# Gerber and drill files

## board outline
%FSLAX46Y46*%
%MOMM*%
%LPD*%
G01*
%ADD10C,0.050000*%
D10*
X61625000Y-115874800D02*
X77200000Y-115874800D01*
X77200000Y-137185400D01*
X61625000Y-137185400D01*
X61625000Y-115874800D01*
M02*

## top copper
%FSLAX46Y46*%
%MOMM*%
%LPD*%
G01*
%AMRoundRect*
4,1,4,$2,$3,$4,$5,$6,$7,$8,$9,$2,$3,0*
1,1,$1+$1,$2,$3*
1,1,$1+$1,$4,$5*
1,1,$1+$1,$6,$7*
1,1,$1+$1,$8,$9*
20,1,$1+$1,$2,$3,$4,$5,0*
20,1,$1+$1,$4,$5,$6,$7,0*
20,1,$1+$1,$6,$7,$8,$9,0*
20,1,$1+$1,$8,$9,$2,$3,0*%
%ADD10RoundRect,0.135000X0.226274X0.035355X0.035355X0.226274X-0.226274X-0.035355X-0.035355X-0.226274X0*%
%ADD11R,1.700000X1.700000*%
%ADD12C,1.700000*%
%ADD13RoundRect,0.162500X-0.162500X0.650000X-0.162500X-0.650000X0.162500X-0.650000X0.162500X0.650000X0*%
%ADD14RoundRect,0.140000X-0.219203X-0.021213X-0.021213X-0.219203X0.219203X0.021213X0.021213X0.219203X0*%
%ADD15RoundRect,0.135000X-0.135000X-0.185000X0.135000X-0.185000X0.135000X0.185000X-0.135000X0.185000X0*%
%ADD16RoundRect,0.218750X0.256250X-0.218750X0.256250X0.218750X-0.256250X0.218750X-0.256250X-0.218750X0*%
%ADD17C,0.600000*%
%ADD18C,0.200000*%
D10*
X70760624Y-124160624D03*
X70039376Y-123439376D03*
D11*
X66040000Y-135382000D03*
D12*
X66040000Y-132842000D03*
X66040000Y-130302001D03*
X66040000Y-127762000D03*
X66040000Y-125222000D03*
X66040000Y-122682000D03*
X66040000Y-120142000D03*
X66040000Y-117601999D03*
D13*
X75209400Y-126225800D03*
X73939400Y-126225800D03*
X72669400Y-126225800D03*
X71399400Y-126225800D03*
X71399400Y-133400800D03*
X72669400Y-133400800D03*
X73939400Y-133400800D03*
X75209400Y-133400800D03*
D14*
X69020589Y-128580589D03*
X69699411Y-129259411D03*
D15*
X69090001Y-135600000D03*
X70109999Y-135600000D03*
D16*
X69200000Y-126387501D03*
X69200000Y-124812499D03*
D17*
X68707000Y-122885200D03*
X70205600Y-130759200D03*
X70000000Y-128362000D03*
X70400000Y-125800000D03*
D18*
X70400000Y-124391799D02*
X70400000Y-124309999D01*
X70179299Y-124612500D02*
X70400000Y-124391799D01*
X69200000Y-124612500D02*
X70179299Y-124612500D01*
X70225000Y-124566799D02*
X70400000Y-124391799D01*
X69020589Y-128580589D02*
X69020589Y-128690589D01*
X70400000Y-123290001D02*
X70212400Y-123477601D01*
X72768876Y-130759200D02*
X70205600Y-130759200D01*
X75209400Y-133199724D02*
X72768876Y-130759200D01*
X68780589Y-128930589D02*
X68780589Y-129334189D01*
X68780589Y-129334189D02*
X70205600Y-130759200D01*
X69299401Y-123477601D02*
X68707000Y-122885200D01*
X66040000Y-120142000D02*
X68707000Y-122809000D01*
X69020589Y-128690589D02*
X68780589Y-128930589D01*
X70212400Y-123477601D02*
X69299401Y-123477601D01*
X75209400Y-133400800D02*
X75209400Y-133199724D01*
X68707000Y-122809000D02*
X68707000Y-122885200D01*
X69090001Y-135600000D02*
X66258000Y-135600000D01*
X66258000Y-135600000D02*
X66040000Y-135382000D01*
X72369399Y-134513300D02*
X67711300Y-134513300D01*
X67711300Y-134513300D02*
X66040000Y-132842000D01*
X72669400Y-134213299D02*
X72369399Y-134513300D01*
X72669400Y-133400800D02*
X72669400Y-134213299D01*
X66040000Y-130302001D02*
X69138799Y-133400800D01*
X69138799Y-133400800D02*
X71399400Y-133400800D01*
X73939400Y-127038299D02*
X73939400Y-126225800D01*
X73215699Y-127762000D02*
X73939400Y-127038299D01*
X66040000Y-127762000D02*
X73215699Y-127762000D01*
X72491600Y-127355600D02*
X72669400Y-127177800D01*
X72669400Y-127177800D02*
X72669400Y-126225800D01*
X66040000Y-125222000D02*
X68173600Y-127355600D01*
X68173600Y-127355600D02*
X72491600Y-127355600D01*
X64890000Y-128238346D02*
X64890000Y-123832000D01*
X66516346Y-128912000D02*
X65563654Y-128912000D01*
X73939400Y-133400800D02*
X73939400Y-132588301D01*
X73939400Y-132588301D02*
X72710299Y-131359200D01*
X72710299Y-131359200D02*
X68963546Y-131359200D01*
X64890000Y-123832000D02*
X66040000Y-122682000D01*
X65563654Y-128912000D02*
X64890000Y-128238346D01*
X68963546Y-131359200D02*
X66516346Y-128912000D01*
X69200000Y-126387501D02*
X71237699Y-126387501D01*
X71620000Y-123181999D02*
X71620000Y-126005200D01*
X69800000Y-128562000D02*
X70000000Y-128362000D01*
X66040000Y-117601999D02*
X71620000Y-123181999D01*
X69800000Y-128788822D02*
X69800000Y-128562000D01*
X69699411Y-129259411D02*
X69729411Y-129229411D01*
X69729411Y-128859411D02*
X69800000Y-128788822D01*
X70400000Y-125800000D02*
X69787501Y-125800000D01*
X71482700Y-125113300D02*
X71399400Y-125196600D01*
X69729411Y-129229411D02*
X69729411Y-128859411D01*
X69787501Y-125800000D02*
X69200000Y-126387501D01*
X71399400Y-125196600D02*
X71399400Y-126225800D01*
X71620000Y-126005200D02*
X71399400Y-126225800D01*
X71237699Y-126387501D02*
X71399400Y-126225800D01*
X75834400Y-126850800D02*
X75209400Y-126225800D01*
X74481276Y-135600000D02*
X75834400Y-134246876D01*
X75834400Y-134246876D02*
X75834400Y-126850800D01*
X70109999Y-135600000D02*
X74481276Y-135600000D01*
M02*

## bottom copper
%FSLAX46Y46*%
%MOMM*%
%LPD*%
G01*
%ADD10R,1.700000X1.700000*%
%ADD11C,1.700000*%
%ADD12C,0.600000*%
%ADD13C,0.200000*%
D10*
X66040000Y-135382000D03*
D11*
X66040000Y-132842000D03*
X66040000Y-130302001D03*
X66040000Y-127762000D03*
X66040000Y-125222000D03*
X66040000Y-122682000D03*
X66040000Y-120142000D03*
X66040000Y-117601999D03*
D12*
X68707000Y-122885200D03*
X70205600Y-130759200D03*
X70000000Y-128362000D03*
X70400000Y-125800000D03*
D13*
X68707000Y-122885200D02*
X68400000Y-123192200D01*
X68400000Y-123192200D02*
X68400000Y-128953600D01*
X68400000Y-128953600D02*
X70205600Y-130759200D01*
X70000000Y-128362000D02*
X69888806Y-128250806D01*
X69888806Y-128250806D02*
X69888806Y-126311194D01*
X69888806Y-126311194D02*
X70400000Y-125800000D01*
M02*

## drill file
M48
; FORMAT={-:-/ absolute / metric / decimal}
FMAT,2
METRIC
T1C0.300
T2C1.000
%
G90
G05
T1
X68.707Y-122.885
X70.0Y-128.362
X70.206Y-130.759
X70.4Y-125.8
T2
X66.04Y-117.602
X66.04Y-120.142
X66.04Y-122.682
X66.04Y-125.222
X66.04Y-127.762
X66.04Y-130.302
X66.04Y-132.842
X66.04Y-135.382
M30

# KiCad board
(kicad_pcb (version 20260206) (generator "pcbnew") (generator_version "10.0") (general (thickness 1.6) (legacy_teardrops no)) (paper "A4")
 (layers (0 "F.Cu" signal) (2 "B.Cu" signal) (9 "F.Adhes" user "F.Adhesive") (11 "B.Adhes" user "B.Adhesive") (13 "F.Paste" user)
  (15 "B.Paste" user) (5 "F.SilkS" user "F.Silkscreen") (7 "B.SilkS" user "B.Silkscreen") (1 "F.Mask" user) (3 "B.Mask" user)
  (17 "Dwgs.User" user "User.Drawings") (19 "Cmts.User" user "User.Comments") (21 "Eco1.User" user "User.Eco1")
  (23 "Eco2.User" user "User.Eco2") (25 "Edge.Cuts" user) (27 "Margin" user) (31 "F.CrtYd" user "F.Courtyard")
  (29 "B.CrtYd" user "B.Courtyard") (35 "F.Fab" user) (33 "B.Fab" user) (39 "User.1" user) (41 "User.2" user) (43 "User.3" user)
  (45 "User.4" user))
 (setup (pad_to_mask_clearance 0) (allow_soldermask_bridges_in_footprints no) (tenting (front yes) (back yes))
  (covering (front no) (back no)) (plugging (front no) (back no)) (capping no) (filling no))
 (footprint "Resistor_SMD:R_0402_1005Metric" (layer "F.Cu") (at 70.4 123.8 135)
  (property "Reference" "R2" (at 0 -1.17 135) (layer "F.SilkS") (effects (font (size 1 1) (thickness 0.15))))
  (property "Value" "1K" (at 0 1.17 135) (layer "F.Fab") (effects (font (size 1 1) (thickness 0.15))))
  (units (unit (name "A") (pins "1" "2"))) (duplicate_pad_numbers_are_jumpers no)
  (pad "1" smd roundrect (at -0.509999 0 135) (size 0.54 0.64) (layers "F.Cu" "F.Mask" "F.Paste") (roundrect_rratio 0.25) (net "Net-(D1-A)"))
  (pad "2" smd roundrect (at 0.509999 0 135) (size 0.54 0.64) (layers "F.Cu" "F.Mask" "F.Paste") (roundrect_rratio 0.25) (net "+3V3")))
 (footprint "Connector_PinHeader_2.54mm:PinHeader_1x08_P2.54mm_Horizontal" (layer "F.Cu") (at 66.04 135.382 180)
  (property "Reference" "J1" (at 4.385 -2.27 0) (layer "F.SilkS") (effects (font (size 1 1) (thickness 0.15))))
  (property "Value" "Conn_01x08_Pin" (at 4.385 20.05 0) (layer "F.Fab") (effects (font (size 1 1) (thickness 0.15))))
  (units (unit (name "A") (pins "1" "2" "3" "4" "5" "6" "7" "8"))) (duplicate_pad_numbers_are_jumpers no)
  (pad "1" thru_hole rect (at 0 0 180) (size 1.7 1.7) (drill 1) (layers "*.Cu" "*.Mask") (remove_unused_layers no) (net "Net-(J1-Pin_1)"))
  (pad "2" thru_hole circle (at 0 2.54 180) (size 1.7 1.7) (drill 1) (layers "*.Cu" "*.Mask") (remove_unused_layers no)
   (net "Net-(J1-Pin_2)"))
  (pad "3" thru_hole circle (at 0 5.079999 180) (size 1.7 1.7) (drill 1) (layers "*.Cu" "*.Mask") (remove_unused_layers no)
   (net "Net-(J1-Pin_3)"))
  (pad "4" thru_hole circle (at 0 7.62 180) (size 1.7 1.7) (drill 1) (layers "*.Cu" "*.Mask") (remove_unused_layers no)
   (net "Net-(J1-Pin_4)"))
  (pad "5" thru_hole circle (at 0 10.16 180) (size 1.7 1.7) (drill 1) (layers "*.Cu" "*.Mask") (remove_unused_layers no)
   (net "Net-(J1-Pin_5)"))
  (pad "6" thru_hole circle (at 0 12.7 180) (size 1.7 1.7) (drill 1) (layers "*.Cu" "*.Mask") (remove_unused_layers no)
   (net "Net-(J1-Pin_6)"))
  (pad "7" thru_hole circle (at 0 15.24 180) (size 1.7 1.7) (drill 1) (layers "*.Cu" "*.Mask") (remove_unused_layers no) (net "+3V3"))
  (pad "8" thru_hole circle (at 0 17.780001 180) (size 1.7 1.7) (drill 1) (layers "*.Cu" "*.Mask") (remove_unused_layers no) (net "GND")))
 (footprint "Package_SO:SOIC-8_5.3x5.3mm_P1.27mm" (layer "F.Cu") (at 73.3044 129.8133 -90)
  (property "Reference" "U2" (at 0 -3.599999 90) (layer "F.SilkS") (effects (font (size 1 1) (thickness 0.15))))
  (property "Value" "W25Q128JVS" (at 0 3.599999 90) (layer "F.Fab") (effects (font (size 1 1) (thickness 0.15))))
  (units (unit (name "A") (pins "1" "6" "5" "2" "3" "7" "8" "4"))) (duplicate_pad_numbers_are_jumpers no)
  (pad "1" smd roundrect (at -3.5875 -1.905 270) (size 1.625 0.65) (layers "F.Cu" "F.Mask" "F.Paste") (roundrect_rratio 0.25)
   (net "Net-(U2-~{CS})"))
  (pad "2" smd roundrect (at -3.5875 -0.635 270) (size 1.625 0.65) (layers "F.Cu" "F.Mask" "F.Paste") (roundrect_rratio 0.25)
   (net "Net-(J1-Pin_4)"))
  (pad "3" smd roundrect (at -3.5875 0.635 270) (size 1.625 0.65) (layers "F.Cu" "F.Mask" "F.Paste") (roundrect_rratio 0.25)
   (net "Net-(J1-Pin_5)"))
  (pad "4" smd roundrect (at -3.5875 1.905 270) (size 1.625 0.65) (layers "F.Cu" "F.Mask" "F.Paste") (roundrect_rratio 0.25) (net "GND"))
  (pad "5" smd roundrect (at 3.5875 1.905 270) (size 1.625 0.65) (layers "F.Cu" "F.Mask" "F.Paste") (roundrect_rratio 0.25)
   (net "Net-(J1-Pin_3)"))
  (pad "6" smd roundrect (at 3.5875 0.635 270) (size 1.625 0.65) (layers "F.Cu" "F.Mask" "F.Paste") (roundrect_rratio 0.25)
   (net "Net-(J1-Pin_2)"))
  (pad "7" smd roundrect (at 3.5875 -0.635 270) (size 1.625 0.65) (layers "F.Cu" "F.Mask" "F.Paste") (roundrect_rratio 0.25)
   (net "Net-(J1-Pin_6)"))
  (pad "8" smd roundrect (at 3.5875 -1.905 270) (size 1.625 0.65) (layers "F.Cu" "F.Mask" "F.Paste") (roundrect_rratio 0.25) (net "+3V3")))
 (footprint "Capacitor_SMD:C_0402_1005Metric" (layer "F.Cu") (at 69.36 128.92 -45)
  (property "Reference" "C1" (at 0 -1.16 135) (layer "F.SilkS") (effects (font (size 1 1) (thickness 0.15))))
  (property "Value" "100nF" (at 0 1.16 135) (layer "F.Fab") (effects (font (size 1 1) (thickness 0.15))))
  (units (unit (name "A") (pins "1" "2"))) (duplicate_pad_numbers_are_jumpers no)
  (pad "1" smd roundrect (at -0.48 0 315) (size 0.56 0.62) (layers "F.Cu" "F.Mask" "F.Paste") (roundrect_rratio 0.25) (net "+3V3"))
  (pad "2" smd roundrect (at 0.48 0 315) (size 0.56 0.62) (layers "F.Cu" "F.Mask" "F.Paste") (roundrect_rratio 0.25) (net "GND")))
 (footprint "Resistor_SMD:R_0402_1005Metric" (layer "F.Cu") (at 69.6 135.6)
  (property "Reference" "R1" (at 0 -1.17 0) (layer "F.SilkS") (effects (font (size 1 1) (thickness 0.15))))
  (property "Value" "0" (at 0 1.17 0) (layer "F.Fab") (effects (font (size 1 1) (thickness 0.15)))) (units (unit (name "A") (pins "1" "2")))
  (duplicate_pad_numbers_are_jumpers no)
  (pad "1" smd roundrect (at -0.509999 0) (size 0.54 0.64) (layers "F.Cu" "F.Mask" "F.Paste") (roundrect_rratio 0.25) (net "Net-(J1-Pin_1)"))
  (pad "2" smd roundrect (at 0.509999 0) (size 0.54 0.64) (layers "F.Cu" "F.Mask" "F.Paste") (roundrect_rratio 0.25) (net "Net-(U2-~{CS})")))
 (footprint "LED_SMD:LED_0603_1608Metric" (layer "F.Cu") (at 69.2 125.6 90)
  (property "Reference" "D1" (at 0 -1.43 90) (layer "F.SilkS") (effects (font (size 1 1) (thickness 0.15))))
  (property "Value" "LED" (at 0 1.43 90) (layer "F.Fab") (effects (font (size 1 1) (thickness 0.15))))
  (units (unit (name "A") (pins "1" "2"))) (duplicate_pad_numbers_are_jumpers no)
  (pad "1" smd roundrect (at -0.787501 0 90) (size 0.875 0.95) (layers "F.Cu" "F.Mask" "F.Paste") (roundrect_rratio 0.25) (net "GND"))
  (pad "2" smd roundrect (at 0.787501 0 90) (size 0.875 0.95) (layers "F.Cu" "F.Mask" "F.Paste") (roundrect_rratio 0.25) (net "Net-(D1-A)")))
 (gr_rect (start 61.625 115.8748) (end 77.2 137.1854) (stroke (width 0.05) (type default)) (fill no) (layer "Edge.Cuts"))
 (segment (start 70.4 124.391799) (end 70.4 124.309999) (width 0.2) (layer "F.Cu") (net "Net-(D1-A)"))
 (segment (start 70.179299 124.6125) (end 70.4 124.391799) (width 0.2) (layer "F.Cu") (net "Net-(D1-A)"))
 (segment (start 69.2 124.6125) (end 70.179299 124.6125) (width 0.2) (layer "F.Cu") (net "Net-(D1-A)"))
 (segment (start 70.225 124.566799) (end 70.4 124.391799) (width 0.2) (layer "F.Cu") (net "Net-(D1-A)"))
 (segment (start 69.020589 128.580589) (end 69.020589 128.690589) (width 0.2) (layer "F.Cu") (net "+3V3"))
 (segment (start 70.4 123.290001) (end 70.2124 123.477601) (width 0.2) (layer "F.Cu") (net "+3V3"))
 (segment (start 72.768876 130.7592) (end 70.2056 130.7592) (width 0.2) (layer "F.Cu") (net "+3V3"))
 (segment (start 75.2094 133.199724) (end 72.768876 130.7592) (width 0.2) (layer "F.Cu") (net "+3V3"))
 (segment (start 68.780589 128.930589) (end 68.780589 129.334189) (width 0.2) (layer "F.Cu") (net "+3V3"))
 (segment (start 68.780589 129.334189) (end 70.2056 130.7592) (width 0.2) (layer "F.Cu") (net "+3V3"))
 (segment (start 69.299401 123.477601) (end 68.707 122.8852) (width 0.2) (layer "F.Cu") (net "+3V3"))
 (segment (start 66.04 120.142) (end 68.707 122.809) (width 0.2) (layer "F.Cu") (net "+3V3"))
 (segment (start 69.020589 128.690589) (end 68.780589 128.930589) (width 0.2) (layer "F.Cu") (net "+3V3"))
 (segment (start 70.2124 123.477601) (end 69.299401 123.477601) (width 0.2) (layer "F.Cu") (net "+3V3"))
 (segment (start 75.2094 133.4008) (end 75.2094 133.199724) (width 0.2) (layer "F.Cu") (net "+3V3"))
 (segment (start 68.707 122.809) (end 68.707 122.8852) (width 0.2) (layer "F.Cu") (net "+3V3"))
 (via (at 68.707 122.8852) (size 0.6) (drill 0.3) (layers "F.Cu" "B.Cu") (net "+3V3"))
 (via (at 70.2056 130.7592) (size 0.6) (drill 0.3) (layers "F.Cu" "B.Cu") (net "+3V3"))
 (segment (start 68.707 122.8852) (end 68.4 123.1922) (width 0.2) (layer "B.Cu") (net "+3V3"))
 (segment (start 68.4 123.1922) (end 68.4 128.9536) (width 0.2) (layer "B.Cu") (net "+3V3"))
 (segment (start 68.4 128.9536) (end 70.2056 130.7592) (width 0.2) (layer "B.Cu") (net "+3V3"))
 (segment (start 69.090001 135.6) (end 66.258 135.6) (width 0.2) (layer "F.Cu") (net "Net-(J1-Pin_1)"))
 (segment (start 66.258 135.6) (end 66.04 135.382) (width 0.2) (layer "F.Cu") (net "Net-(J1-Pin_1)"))
 (segment (start 72.369399 134.5133) (end 67.7113 134.5133) (width 0.2) (layer "F.Cu") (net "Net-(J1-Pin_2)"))
 (segment (start 67.7113 134.5133) (end 66.04 132.842) (width 0.2) (layer "F.Cu") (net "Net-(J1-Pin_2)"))
 (segment (start 72.6694 134.213299) (end 72.369399 134.5133) (width 0.2) (layer "F.Cu") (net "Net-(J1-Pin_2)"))
 (segment (start 72.6694 133.4008) (end 72.6694 134.213299) (width 0.2) (layer "F.Cu") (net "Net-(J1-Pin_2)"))
 (segment (start 66.04 130.302001) (end 69.138799 133.4008) (width 0.2) (layer "F.Cu") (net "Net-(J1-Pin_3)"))
 (segment (start 69.138799 133.4008) (end 71.3994 133.4008) (width 0.2) (layer "F.Cu") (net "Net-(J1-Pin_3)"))
 (segment (start 73.9394 127.038299) (end 73.9394 126.2258) (width 0.2) (layer "F.Cu") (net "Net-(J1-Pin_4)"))
 (segment (start 73.215699 127.762) (end 73.9394 127.038299) (width 0.2) (layer "F.Cu") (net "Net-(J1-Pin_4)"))
 (segment (start 66.04 127.762) (end 73.215699 127.762) (width 0.2) (layer "F.Cu") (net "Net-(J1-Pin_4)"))
 (segment (start 72.4916 127.3556) (end 72.6694 127.1778) (width 0.2) (layer "F.Cu") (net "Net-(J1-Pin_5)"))
 (segment (start 72.6694 127.1778) (end 72.6694 126.2258) (width 0.2) (layer "F.Cu") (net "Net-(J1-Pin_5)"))
 (segment (start 66.04 125.222) (end 68.1736 127.3556) (width 0.2) (layer "F.Cu") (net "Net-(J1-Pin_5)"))
 (segment (start 68.1736 127.3556) (end 72.4916 127.3556) (width 0.2) (layer "F.Cu") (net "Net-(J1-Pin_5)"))
 (segment (start 64.89 128.238346) (end 64.89 123.832) (width 0.2) (layer "F.Cu") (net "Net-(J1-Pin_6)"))
 (segment (start 66.516346 128.912) (end 65.563654 128.912) (width 0.2) (layer "F.Cu") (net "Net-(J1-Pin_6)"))
 (segment (start 73.9394 133.4008) (end 73.9394 132.588301) (width 0.2) (layer "F.Cu") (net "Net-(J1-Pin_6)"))
 (segment (start 73.9394 132.588301) (end 72.710299 131.3592) (width 0.2) (layer "F.Cu") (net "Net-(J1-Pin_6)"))
 (segment (start 72.710299 131.3592) (end 68.963546 131.3592) (width 0.2) (layer "F.Cu") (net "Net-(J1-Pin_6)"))
 (segment (start 64.89 123.832) (end 66.04 122.682) (width 0.2) (layer "F.Cu") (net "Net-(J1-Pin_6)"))
 (segment (start 65.563654 128.912) (end 64.89 128.238346) (width 0.2) (layer "F.Cu") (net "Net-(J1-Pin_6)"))
 (segment (start 68.963546 131.3592) (end 66.516346 128.912) (width 0.2) (layer "F.Cu") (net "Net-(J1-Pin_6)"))
 (segment (start 69.2 126.387501) (end 71.237699 126.387501) (width 0.2) (layer "F.Cu") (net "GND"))
 (segment (start 71.62 123.181999) (end 71.62 126.0052) (width 0.2) (layer "F.Cu") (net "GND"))
 (segment (start 69.8 128.562) (end 70 128.362) (width 0.2) (layer "F.Cu") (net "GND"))
 (segment (start 66.04 117.601999) (end 71.62 123.181999) (width 0.2) (layer "F.Cu") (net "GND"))
 (segment (start 69.8 128.788822) (end 69.8 128.562) (width 0.2) (layer "F.Cu") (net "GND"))
 (segment (start 69.699411 129.259411) (end 69.729411 129.229411) (width 0.2) (layer "F.Cu") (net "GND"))
 (segment (start 69.729411 128.859411) (end 69.8 128.788822) (width 0.2) (layer "F.Cu") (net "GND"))
 (segment (start 70.4 125.8) (end 69.787501 125.8) (width 0.2) (layer "F.Cu") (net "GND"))
 (segment (start 71.4827 125.1133) (end 71.3994 125.1966) (width 0.2) (layer "F.Cu") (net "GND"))
 (segment (start 69.729411 129.229411) (end 69.729411 128.859411) (width 0.2) (layer "F.Cu") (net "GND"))
 (segment (start 69.787501 125.8) (end 69.2 126.387501) (width 0.2) (layer "F.Cu") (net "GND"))
 (segment (start 71.3994 125.1966) (end 71.3994 126.2258) (width 0.2) (layer "F.Cu") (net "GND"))
 (segment (start 71.62 126.0052) (end 71.3994 126.2258) (width 0.2) (layer "F.Cu") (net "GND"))
 (segment (start 71.237699 126.387501) (end 71.3994 126.2258) (width 0.2) (layer "F.Cu") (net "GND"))
 (via (at 70 128.362) (size 0.6) (drill 0.3) (layers "F.Cu" "B.Cu") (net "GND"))
 (via (at 70.4 125.8) (size 0.6) (drill 0.3) (layers "F.Cu" "B.Cu") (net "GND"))
 (segment (start 70 128.362) (end 69.888806 128.250806) (width 0.2) (layer "B.Cu") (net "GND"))
 (segment (start 69.888806 128.250806) (end 69.888806 126.311194) (width 0.2) (layer "B.Cu") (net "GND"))
 (segment (start 69.888806 126.311194) (end 70.4 125.8) (width 0.2) (layer "B.Cu") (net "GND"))
 (segment (start 75.8344 126.8508) (end 75.2094 126.2258) (width 0.2) (layer "F.Cu") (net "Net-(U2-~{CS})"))
 (segment (start 74.481276 135.6) (end 75.8344 134.246876) (width 0.2) (layer "F.Cu") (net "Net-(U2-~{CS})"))
 (segment (start 75.8344 134.246876) (end 75.8344 126.8508) (width 0.2) (layer "F.Cu") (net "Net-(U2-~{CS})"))
 (segment (start 70.109999 135.6) (end 74.481276 135.6) (width 0.2) (layer "F.Cu") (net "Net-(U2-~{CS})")))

